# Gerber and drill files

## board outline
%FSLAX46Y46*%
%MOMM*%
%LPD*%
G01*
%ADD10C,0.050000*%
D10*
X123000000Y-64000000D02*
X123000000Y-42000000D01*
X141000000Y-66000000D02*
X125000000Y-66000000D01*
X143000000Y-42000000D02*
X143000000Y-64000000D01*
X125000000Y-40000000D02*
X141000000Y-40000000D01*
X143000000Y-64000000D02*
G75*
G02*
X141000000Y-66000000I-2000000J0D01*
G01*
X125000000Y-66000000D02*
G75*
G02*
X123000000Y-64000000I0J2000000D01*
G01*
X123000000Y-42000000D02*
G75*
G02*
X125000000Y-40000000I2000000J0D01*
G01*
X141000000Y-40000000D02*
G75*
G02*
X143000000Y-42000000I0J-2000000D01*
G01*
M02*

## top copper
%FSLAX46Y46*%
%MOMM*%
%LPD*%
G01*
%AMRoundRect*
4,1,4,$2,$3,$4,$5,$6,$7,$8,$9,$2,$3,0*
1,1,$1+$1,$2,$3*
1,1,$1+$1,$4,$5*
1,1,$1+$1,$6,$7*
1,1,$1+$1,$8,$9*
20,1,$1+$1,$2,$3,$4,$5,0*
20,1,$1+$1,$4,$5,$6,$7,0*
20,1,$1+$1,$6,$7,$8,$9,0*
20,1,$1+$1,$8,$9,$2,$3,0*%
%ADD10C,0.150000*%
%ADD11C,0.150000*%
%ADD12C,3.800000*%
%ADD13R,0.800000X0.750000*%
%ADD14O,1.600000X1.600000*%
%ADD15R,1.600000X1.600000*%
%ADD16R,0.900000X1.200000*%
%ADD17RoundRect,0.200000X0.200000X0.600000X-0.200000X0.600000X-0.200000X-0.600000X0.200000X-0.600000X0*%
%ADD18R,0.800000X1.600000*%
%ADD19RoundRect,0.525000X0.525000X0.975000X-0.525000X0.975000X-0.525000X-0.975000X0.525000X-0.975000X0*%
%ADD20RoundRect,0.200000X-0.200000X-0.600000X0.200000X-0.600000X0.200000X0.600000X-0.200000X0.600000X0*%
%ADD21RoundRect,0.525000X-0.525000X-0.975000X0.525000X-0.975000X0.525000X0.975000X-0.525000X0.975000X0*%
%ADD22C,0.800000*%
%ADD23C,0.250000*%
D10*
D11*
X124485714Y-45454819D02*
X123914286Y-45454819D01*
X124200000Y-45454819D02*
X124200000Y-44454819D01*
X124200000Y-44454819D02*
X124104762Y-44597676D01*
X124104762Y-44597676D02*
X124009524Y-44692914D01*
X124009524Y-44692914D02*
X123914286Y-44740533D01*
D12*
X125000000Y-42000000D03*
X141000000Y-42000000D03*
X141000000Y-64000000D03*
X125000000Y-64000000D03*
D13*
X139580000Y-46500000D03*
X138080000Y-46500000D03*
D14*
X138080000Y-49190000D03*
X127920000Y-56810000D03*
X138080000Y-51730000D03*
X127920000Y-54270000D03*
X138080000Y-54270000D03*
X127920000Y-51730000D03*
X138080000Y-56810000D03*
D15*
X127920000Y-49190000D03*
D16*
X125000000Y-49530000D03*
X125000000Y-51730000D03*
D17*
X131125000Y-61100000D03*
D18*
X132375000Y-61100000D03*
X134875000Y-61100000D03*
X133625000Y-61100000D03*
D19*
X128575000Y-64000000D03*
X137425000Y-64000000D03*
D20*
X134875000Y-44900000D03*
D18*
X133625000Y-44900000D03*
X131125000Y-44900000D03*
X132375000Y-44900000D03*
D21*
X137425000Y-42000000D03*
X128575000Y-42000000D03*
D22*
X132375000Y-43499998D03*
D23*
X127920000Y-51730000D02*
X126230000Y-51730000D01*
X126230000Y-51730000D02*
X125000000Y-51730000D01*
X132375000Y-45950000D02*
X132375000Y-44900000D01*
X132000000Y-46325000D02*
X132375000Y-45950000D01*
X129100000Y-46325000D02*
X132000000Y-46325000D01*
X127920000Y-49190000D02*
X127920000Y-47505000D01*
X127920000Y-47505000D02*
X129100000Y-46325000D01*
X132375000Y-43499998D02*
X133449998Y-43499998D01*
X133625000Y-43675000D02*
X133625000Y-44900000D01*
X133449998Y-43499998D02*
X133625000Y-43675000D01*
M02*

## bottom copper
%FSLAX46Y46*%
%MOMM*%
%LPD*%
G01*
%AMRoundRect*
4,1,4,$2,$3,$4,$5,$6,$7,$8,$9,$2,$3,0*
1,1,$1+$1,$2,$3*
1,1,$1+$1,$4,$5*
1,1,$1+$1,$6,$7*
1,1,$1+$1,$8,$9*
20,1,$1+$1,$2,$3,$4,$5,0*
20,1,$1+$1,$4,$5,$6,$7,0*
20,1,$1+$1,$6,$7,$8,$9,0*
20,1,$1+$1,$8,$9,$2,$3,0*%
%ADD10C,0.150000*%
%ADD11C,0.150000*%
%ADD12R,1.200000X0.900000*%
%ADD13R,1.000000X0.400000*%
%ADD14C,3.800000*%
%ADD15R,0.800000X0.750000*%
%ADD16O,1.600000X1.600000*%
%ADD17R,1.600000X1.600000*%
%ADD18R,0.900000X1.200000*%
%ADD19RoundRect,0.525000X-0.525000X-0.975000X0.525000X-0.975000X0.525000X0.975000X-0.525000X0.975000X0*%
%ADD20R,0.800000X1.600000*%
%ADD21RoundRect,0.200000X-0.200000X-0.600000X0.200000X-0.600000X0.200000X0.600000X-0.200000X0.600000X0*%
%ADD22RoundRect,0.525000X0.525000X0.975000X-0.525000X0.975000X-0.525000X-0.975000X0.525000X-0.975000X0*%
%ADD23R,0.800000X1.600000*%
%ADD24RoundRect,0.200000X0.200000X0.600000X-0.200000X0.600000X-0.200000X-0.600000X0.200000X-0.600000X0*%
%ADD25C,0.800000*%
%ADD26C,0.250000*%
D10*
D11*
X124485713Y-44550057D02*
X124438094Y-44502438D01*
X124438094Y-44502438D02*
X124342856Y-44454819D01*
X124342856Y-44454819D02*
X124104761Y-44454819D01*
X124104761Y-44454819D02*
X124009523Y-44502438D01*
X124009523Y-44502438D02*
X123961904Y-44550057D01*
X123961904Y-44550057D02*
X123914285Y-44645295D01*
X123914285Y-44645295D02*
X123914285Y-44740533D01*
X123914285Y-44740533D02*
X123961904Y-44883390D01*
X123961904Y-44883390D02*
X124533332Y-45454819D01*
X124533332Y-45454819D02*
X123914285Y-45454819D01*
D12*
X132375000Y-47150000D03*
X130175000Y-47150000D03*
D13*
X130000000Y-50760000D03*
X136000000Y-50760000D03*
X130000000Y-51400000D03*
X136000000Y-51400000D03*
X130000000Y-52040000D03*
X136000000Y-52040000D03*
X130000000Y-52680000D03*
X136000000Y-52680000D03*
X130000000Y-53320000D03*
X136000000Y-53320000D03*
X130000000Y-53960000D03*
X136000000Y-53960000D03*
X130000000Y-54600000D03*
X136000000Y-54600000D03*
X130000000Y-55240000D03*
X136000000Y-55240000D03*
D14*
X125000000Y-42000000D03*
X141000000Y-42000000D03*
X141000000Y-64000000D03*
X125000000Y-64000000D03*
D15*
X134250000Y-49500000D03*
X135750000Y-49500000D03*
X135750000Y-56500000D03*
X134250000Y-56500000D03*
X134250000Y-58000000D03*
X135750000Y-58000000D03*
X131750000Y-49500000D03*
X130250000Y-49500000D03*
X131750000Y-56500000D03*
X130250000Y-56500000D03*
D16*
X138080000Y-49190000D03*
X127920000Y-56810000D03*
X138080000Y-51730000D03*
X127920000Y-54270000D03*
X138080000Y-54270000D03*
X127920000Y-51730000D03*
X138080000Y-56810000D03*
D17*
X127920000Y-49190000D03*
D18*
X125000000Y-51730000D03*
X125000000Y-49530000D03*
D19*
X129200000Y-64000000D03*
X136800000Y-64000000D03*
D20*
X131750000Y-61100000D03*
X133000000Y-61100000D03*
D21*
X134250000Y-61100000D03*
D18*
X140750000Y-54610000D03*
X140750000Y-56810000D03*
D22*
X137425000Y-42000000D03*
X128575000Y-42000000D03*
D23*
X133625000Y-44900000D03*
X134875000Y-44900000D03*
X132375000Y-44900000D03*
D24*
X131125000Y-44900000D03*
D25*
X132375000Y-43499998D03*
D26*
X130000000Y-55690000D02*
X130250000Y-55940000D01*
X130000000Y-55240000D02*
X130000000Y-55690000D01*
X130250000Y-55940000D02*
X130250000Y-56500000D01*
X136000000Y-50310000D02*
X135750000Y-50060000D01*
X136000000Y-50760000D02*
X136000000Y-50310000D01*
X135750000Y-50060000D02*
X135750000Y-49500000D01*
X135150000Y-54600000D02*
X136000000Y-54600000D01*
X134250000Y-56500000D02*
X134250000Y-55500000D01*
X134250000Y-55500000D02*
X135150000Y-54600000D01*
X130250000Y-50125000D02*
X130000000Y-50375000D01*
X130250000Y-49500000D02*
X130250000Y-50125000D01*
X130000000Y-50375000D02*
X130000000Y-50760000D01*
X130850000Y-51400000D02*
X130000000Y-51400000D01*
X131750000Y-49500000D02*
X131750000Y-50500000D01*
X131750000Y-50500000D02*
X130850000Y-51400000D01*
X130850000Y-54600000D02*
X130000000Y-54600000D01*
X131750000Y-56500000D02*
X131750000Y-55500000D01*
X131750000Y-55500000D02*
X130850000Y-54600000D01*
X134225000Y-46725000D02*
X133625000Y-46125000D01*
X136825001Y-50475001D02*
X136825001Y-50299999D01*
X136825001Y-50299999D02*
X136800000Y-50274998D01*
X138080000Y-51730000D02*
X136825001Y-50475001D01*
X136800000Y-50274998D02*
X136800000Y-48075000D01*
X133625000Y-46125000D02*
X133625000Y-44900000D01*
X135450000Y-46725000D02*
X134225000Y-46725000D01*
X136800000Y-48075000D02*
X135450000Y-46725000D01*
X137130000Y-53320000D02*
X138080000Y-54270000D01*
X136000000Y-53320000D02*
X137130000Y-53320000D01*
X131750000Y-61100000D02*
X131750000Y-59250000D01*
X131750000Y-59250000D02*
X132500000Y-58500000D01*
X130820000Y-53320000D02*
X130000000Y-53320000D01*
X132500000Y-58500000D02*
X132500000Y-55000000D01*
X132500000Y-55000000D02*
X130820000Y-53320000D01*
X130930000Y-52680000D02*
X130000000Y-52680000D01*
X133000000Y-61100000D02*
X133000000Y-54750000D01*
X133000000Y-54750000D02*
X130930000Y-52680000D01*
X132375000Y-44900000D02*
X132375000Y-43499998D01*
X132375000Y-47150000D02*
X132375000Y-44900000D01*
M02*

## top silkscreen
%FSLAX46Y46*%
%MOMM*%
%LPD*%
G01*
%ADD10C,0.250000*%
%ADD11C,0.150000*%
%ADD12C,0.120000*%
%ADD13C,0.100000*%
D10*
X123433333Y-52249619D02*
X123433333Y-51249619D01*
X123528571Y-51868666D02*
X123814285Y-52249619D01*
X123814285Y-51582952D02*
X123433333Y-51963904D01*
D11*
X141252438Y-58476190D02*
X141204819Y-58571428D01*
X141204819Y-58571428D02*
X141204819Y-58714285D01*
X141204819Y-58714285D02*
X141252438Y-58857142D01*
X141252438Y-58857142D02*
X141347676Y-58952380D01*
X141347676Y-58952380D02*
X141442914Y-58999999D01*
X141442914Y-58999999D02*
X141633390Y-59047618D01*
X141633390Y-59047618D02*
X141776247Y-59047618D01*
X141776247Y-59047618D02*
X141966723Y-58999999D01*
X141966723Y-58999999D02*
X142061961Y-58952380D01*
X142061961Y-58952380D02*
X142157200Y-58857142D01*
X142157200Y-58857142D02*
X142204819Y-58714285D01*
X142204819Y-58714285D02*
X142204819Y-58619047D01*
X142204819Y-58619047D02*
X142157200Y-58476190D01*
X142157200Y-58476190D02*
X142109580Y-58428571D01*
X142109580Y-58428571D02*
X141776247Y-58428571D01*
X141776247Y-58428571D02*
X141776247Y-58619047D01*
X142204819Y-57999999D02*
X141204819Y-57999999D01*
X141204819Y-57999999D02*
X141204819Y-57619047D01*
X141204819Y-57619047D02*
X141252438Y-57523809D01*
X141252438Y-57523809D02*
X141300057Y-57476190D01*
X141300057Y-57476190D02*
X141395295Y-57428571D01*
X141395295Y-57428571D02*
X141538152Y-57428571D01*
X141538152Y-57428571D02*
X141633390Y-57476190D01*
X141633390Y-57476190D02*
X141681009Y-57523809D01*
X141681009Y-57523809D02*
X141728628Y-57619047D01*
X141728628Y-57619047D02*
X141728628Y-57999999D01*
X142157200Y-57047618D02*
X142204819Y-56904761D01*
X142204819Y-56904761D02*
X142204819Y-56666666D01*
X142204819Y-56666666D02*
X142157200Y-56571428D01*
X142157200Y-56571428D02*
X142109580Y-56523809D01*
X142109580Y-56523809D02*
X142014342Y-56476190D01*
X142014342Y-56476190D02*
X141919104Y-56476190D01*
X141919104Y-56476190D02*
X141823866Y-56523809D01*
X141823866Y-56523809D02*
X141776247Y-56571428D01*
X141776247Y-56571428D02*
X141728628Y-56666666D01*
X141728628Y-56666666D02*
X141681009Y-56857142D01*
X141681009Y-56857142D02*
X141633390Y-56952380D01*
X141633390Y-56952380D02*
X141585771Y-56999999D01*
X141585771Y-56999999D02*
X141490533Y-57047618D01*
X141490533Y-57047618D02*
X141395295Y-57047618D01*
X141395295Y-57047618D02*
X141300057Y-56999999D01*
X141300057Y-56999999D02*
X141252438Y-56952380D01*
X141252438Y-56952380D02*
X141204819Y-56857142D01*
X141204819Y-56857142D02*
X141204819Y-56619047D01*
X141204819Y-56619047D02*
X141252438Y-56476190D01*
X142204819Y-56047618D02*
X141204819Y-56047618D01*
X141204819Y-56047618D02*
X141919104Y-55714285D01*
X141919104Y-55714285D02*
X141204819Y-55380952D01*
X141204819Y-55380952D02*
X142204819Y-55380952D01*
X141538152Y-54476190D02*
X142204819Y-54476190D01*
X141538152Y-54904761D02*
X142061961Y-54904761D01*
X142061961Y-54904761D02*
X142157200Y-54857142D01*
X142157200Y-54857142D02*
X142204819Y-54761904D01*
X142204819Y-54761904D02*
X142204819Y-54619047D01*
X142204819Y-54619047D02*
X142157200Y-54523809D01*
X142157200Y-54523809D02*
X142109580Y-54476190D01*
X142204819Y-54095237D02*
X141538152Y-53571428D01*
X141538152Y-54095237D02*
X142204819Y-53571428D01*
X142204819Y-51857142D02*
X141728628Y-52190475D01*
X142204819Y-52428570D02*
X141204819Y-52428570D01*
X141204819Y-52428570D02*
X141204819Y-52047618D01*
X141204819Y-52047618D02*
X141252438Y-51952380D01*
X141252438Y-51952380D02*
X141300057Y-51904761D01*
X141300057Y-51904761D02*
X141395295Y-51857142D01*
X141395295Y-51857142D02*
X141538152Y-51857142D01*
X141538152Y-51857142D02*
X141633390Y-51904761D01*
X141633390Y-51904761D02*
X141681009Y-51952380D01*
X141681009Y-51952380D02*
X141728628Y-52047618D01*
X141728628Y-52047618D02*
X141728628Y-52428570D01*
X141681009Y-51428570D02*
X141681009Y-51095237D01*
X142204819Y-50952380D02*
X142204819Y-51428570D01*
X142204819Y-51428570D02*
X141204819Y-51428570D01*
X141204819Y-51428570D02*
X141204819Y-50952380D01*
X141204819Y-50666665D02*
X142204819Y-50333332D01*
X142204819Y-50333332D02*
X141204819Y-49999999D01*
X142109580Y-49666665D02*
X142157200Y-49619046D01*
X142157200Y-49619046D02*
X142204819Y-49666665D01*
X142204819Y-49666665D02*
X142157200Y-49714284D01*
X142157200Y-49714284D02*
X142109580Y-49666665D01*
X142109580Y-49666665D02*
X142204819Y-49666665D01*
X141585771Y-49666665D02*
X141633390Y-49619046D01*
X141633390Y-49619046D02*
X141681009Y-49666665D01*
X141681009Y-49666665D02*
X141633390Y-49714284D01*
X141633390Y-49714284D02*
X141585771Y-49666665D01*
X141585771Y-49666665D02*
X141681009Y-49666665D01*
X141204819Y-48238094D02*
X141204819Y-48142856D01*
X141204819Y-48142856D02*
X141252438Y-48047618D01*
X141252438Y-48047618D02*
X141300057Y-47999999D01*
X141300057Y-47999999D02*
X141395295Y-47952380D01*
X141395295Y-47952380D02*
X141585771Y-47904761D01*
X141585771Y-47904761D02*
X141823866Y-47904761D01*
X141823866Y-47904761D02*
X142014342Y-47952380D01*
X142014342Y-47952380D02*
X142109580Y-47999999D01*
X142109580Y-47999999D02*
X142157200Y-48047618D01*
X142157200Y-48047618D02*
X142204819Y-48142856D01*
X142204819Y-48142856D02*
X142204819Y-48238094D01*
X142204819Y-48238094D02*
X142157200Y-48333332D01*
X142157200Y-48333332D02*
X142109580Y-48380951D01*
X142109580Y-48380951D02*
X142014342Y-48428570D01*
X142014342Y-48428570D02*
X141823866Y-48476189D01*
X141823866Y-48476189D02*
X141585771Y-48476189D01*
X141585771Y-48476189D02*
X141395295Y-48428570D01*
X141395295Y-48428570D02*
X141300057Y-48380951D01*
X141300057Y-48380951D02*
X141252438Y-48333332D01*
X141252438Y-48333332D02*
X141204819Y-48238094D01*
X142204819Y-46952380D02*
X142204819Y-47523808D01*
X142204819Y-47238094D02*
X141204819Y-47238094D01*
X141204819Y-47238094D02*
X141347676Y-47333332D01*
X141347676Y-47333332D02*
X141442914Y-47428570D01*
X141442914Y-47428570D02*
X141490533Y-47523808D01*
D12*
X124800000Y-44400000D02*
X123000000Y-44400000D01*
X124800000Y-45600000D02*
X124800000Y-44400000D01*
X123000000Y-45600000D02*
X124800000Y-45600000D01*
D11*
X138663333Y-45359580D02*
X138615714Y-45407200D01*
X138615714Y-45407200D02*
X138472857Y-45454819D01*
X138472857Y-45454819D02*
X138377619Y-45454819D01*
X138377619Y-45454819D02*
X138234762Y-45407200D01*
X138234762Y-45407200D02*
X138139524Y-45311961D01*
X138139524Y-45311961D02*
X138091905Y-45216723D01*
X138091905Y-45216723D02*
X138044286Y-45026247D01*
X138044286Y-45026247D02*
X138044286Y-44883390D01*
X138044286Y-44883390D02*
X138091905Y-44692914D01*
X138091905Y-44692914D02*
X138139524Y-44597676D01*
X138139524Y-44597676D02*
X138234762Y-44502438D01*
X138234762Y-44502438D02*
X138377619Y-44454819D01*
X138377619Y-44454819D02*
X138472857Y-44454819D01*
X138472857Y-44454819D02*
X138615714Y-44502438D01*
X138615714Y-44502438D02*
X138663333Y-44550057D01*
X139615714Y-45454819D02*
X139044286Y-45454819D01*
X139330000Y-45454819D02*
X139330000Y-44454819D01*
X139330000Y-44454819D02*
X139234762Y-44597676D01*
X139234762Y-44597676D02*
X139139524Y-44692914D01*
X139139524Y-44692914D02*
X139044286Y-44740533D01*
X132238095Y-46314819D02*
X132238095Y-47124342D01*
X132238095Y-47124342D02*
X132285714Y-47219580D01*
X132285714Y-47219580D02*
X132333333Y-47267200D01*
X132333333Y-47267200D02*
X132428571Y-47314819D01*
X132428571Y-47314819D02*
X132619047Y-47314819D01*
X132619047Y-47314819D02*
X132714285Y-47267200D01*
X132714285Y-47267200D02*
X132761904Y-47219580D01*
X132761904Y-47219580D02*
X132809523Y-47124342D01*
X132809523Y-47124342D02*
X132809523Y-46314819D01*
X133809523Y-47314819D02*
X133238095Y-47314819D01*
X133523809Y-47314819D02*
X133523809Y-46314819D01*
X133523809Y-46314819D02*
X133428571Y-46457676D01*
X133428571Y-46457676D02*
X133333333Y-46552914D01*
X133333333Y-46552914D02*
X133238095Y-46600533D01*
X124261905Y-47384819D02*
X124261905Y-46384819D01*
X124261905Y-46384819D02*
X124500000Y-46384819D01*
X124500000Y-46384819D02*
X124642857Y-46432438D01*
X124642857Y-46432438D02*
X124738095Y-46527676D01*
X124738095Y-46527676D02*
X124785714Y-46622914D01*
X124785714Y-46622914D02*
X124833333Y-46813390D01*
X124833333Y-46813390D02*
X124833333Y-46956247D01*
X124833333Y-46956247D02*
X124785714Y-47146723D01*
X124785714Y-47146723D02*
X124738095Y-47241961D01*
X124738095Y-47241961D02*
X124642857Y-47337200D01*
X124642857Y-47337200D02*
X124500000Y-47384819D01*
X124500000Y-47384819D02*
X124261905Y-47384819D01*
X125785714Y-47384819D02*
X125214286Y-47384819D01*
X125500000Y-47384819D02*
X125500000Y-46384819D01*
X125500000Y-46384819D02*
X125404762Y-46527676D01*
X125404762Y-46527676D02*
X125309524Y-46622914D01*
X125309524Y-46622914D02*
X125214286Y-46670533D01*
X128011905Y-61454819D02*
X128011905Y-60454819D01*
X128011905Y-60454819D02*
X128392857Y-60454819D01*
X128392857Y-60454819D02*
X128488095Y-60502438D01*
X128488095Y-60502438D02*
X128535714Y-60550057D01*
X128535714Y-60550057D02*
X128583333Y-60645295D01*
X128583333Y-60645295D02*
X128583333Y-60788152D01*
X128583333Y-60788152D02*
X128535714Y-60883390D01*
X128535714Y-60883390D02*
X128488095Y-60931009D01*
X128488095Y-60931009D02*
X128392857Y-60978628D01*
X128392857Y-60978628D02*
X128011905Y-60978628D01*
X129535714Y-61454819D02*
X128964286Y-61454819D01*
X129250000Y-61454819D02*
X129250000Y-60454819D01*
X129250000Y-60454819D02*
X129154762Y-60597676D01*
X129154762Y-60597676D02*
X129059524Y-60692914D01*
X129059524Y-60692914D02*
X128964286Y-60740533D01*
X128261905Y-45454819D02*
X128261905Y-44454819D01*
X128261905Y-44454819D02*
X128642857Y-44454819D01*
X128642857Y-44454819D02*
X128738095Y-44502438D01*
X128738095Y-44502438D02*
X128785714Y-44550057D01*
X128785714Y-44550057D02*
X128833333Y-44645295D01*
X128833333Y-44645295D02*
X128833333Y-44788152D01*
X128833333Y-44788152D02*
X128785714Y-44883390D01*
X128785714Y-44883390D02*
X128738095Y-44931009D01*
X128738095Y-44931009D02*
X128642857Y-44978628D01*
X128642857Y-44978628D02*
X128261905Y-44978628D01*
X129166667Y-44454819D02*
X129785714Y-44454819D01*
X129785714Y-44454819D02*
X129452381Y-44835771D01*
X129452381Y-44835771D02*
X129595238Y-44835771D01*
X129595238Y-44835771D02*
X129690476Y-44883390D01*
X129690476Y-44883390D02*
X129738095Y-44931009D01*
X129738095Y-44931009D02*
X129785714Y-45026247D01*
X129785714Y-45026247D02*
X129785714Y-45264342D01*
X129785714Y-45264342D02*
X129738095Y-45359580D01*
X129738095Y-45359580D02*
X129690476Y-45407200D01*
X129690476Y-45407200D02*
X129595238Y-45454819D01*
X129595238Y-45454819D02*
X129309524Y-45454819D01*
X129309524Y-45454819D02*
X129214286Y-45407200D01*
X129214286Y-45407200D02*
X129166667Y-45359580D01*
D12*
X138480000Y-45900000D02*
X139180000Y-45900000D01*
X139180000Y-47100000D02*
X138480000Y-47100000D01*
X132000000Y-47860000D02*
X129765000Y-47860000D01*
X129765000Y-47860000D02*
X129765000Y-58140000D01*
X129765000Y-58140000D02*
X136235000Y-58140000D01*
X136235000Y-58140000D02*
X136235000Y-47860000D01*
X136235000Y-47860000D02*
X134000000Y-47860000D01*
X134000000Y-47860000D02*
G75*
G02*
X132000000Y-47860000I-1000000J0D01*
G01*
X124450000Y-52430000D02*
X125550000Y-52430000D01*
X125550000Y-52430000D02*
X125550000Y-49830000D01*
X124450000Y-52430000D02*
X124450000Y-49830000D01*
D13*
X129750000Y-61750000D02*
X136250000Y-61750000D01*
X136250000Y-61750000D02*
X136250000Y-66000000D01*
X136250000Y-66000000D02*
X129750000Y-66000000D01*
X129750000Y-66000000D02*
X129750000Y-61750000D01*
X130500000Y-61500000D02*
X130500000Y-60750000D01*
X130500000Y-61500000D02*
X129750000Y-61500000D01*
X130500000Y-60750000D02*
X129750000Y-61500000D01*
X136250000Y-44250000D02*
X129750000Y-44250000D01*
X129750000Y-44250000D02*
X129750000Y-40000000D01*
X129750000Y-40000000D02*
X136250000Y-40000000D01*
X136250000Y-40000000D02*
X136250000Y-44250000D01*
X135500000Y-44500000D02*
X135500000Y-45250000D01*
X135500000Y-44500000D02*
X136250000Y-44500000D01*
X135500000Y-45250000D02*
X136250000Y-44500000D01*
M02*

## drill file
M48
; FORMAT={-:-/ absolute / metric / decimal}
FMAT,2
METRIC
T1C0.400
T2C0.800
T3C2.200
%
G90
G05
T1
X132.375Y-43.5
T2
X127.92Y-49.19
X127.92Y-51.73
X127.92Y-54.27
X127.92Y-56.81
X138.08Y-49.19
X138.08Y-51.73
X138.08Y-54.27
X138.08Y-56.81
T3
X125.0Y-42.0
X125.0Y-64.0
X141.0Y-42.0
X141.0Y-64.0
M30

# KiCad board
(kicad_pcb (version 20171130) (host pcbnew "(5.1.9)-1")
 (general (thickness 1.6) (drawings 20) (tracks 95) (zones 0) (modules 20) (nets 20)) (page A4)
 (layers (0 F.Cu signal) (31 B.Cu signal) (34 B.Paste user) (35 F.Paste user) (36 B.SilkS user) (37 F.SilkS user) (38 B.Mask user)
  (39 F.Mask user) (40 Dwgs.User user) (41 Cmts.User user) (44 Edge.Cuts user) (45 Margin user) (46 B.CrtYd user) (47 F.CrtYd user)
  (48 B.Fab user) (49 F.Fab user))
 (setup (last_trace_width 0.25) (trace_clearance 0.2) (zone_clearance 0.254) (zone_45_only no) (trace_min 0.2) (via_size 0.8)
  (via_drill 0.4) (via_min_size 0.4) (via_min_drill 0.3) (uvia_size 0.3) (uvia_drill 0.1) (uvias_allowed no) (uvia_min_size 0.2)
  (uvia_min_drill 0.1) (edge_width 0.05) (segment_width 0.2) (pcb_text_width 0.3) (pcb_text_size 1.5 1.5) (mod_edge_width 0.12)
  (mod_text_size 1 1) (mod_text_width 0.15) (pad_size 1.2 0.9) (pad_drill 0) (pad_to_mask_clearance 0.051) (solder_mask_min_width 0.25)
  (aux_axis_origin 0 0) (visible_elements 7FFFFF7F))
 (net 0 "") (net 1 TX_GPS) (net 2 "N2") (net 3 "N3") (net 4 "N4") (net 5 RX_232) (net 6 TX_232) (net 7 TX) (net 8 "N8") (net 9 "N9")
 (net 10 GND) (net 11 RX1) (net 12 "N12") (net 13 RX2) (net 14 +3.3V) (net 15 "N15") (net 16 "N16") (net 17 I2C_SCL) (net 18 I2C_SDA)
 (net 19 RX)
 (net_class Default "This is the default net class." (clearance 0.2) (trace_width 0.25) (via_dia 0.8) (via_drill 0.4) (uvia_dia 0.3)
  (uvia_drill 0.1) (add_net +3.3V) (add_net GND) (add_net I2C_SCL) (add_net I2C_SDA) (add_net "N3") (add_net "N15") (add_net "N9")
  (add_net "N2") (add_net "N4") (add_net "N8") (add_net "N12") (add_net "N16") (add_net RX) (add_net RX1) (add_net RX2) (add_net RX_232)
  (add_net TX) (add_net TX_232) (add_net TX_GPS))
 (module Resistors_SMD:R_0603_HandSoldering (layer B.Cu) (at 131.275 47.15 180)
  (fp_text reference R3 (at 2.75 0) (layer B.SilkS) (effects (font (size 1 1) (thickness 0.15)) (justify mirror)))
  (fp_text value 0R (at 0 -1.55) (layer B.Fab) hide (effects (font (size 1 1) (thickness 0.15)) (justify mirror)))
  (pad 1 smd rect (at -1.1 0 180) (size 1.2 0.9) (layers B.Cu B.Paste B.Mask) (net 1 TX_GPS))
  (pad 2 smd rect (at 1.1 0 180) (size 1.2 0.9) (layers B.Cu B.Paste B.Mask)))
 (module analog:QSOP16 (layer B.Cu) (at 133 53 270) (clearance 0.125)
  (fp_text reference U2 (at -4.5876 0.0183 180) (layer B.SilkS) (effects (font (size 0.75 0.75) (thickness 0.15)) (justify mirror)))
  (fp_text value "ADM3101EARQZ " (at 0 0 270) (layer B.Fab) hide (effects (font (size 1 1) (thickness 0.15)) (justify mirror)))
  (pad 16 smd rect (at -2.24 3 270) (size 0.4 1) (layers B.Cu B.Paste B.Mask) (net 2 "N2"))
  (pad 1 smd rect (at -2.24 -3 270) (size 0.4 1) (layers B.Cu B.Paste B.Mask) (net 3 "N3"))
  (pad 15 smd rect (at -1.6 3 270) (size 0.4 1) (layers B.Cu B.Paste B.Mask) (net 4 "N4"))
  (pad 2 smd rect (at -1.6 -3 270) (size 0.4 1) (layers B.Cu B.Paste B.Mask))
  (pad 14 smd rect (at -0.96 3 270) (size 0.4 1) (layers B.Cu B.Paste B.Mask))
  (pad 3 smd rect (at -0.96 -3 270) (size 0.4 1) (layers B.Cu B.Paste B.Mask))
  (pad 13 smd rect (at -0.32 3 270) (size 0.4 1) (layers B.Cu B.Paste B.Mask) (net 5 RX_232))
  (pad 4 smd rect (at -0.32 -3 270) (size 0.4 1) (layers B.Cu B.Paste B.Mask))
  (pad 12 smd rect (at 0.32 3 270) (size 0.4 1) (layers B.Cu B.Paste B.Mask) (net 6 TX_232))
  (pad 5 smd rect (at 0.32 -3 270) (size 0.4 1) (layers B.Cu B.Paste B.Mask) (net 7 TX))
  (pad 11 smd rect (at 0.96 3 270) (size 0.4 1) (layers B.Cu B.Paste B.Mask))
  (pad 6 smd rect (at 0.96 -3 270) (size 0.4 1) (layers B.Cu B.Paste B.Mask))
  (pad 10 smd rect (at 1.6 3 270) (size 0.4 1) (layers B.Cu B.Paste B.Mask) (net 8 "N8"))
  (pad 7 smd rect (at 1.6 -3 270) (size 0.4 1) (layers B.Cu B.Paste B.Mask) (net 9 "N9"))
  (pad 9 smd rect (at 2.24 3 270) (size 0.4 1) (layers B.Cu B.Paste B.Mask) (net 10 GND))
  (pad 8 smd rect (at 2.24 -3 270) (size 0.4 1) (layers B.Cu B.Paste B.Mask)))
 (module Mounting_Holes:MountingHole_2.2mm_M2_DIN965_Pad (layer F.Cu) (at 125 42)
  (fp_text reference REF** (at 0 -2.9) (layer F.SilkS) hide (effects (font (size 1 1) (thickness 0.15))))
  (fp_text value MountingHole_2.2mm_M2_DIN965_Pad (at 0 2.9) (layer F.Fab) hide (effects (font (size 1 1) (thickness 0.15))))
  (pad 1 thru_hole circle (at 0 0) (size 3.8 3.8) (drill 2.2) (layers *.Cu *.Mask)))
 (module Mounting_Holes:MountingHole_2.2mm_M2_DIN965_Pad (layer F.Cu) (at 141 42)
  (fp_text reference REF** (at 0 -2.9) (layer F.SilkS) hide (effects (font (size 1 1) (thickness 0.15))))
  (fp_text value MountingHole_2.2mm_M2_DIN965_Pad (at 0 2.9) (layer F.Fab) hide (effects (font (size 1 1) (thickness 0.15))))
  (pad 1 thru_hole circle (at 0 0) (size 3.8 3.8) (drill 2.2) (layers *.Cu *.Mask)))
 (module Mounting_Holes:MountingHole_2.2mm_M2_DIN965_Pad (layer F.Cu) (at 141 64)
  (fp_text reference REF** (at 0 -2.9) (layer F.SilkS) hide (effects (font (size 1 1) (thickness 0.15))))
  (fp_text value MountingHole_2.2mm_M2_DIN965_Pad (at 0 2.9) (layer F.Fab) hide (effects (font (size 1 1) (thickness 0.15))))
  (pad 1 thru_hole circle (at 0 0) (size 3.8 3.8) (drill 2.2) (layers *.Cu *.Mask)))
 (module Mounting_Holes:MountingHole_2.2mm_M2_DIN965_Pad (layer F.Cu) (at 125 64)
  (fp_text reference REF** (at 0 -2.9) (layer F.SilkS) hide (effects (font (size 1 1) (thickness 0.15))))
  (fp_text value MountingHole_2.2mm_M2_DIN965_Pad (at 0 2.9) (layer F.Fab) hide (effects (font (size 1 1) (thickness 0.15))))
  (pad 1 thru_hole circle (at 0 0) (size 3.8 3.8) (drill 2.2) (layers *.Cu *.Mask)))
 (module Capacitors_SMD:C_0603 (layer F.Cu) (at 138.83 46.5)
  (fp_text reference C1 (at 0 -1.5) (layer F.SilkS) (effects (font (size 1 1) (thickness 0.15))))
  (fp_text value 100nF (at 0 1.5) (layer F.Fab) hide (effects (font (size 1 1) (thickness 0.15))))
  (fp_line (start -0.35 -0.6) (end 0.35 -0.6) (layer F.SilkS) (width 0.12))
  (fp_line (start 0.35 0.6) (end -0.35 0.6) (layer F.SilkS) (width 0.12))
  (pad 2 smd rect (at 0.75 0) (size 0.8 0.75) (layers F.Cu F.Paste F.Mask))
  (pad 1 smd rect (at -0.75 0) (size 0.8 0.75) (layers F.Cu F.Paste F.Mask)))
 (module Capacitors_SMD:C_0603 (layer B.Cu) (at 135 49.5 180)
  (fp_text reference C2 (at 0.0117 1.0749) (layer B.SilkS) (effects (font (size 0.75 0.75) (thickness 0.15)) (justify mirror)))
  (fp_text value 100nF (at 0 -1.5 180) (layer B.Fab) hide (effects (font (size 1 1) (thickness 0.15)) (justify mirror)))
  (pad 2 smd rect (at 0.75 0 180) (size 0.8 0.75) (layers B.Cu B.Paste B.Mask))
  (pad 1 smd rect (at -0.75 0 180) (size 0.8 0.75) (layers B.Cu B.Paste B.Mask) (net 3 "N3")))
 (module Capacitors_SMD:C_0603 (layer B.Cu) (at 135 56.5)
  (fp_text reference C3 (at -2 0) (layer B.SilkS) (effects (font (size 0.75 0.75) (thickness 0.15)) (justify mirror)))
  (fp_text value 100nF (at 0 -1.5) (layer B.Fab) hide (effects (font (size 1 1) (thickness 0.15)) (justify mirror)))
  (pad 2 smd rect (at 0.75 0) (size 0.8 0.75) (layers B.Cu B.Paste B.Mask))
  (pad 1 smd rect (at -0.75 0) (size 0.8 0.75) (layers B.Cu B.Paste B.Mask) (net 9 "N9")))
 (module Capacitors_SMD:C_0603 (layer B.Cu) (at 135 58 180)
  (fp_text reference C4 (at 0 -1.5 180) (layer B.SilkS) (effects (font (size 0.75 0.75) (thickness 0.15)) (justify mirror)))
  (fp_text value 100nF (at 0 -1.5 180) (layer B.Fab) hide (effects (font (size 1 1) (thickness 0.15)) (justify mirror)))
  (pad 2 smd rect (at 0.75 0 180) (size 0.8 0.75) (layers B.Cu B.Paste B.Mask))
  (pad 1 smd rect (at -0.75 0 180) (size 0.8 0.75) (layers B.Cu B.Paste B.Mask)))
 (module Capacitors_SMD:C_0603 (layer B.Cu) (at 131 49.5)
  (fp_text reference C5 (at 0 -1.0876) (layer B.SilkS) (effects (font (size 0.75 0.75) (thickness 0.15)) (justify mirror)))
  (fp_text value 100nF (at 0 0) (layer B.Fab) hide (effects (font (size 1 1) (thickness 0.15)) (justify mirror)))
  (pad 2 smd rect (at 0.75 0) (size 0.8 0.75) (layers B.Cu B.Paste B.Mask) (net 4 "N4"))
  (pad 1 smd rect (at -0.75 0) (size 0.8 0.75) (layers B.Cu B.Paste B.Mask) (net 2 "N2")))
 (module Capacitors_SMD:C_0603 (layer B.Cu) (at 131 56.5)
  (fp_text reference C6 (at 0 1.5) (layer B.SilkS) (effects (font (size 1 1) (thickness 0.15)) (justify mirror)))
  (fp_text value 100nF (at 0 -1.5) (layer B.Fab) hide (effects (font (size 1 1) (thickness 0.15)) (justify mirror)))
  (pad 2 smd rect (at 0.75 0) (size 0.8 0.75) (layers B.Cu B.Paste B.Mask) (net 8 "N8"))
  (pad 1 smd rect (at -0.75 0) (size 0.8 0.75) (layers B.Cu B.Paste B.Mask) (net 10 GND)))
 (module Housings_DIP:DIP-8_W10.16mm (layer F.Cu) (at 133 53)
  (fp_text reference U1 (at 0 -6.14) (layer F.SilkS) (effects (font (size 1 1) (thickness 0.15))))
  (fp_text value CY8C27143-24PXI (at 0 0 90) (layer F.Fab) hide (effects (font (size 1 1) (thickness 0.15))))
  (fp_line (start -1 -5.14) (end -3.235 -5.14) (layer F.SilkS) (width 0.12))
  (fp_line (start -3.235 -5.14) (end -3.235 5.14) (layer F.SilkS) (width 0.12))
  (fp_line (start -3.235 5.14) (end 3.235 5.14) (layer F.SilkS) (width 0.12))
  (fp_line (start 3.235 5.14) (end 3.235 -5.14) (layer F.SilkS) (width 0.12))
  (fp_line (start 3.235 -5.14) (end 1 -5.14) (layer F.SilkS) (width 0.12))
  (fp_arc (start 0 -5.14) (end -1 -5.14) (angle -180) (layer F.SilkS) (width 0.12))
  (pad 8 thru_hole oval (at 5.08 -3.81) (size 1.6 1.6) (drill 0.8) (layers *.Cu *.Mask))
  (pad 4 thru_hole oval (at -5.08 3.81) (size 1.6 1.6) (drill 0.8) (layers *.Cu *.Mask))
  (pad 7 thru_hole oval (at 5.08 -1.27) (size 1.6 1.6) (drill 0.8) (layers *.Cu *.Mask) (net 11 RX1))
  (pad 3 thru_hole oval (at -5.08 1.27) (size 1.6 1.6) (drill 0.8) (layers *.Cu *.Mask))
  (pad 6 thru_hole oval (at 5.08 1.27) (size 1.6 1.6) (drill 0.8) (layers *.Cu *.Mask) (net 7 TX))
  (pad 2 thru_hole oval (at -5.08 -1.27) (size 1.6 1.6) (drill 0.8) (layers *.Cu *.Mask) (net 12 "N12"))
  (pad 5 thru_hole oval (at 5.08 3.81) (size 1.6 1.6) (drill 0.8) (layers *.Cu *.Mask))
  (pad 1 thru_hole rect (at -5.08 -3.81) (size 1.6 1.6) (drill 0.8) (layers *.Cu *.Mask) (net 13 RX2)))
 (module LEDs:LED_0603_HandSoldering (layer F.Cu) (at 125 50.63 90)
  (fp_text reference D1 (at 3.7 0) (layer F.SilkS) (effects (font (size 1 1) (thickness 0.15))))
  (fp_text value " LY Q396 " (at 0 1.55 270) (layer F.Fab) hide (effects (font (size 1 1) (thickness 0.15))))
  (fp_line (start -1.8 -0.55) (end -1.8 0.55) (layer F.SilkS) (width 0.12))
  (fp_line (start -1.8 0.55) (end 0.8 0.55) (layer F.SilkS) (width 0.12))
  (fp_line (start -1.8 -0.55) (end 0.8 -0.55) (layer F.SilkS) (width 0.12))
  (pad 2 smd rect (at 1.1 0 90) (size 1.2 0.9) (layers F.Cu F.Paste F.Mask))
  (pad 1 smd rect (at -1.1 0 90) (size 1.2 0.9) (layers F.Cu F.Paste F.Mask) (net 12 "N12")))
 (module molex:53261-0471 (layer F.Cu) (at 133 64 180) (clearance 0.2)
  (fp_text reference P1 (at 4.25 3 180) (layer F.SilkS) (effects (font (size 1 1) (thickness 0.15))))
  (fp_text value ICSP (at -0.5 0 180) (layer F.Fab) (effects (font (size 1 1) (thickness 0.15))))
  (fp_line (start 3.25 2.25) (end -3.25 2.25) (layer F.SilkS) (width 0.1))
  (fp_line (start -3.25 2.25) (end -3.25 -2) (layer F.SilkS) (width 0.1))
  (fp_line (start -3.25 -2) (end 3.25 -2) (layer F.SilkS) (width 0.1))
  (fp_line (start 3.25 -2) (end 3.25 2.25) (layer F.SilkS) (width 0.1))
  (fp_line (start 2.5 2.5) (end 2.5 3.25) (layer F.SilkS) (width 0.1))
  (fp_line (start 2.5 2.5) (end 3.25 2.5) (layer F.SilkS) (width 0.1))
  (fp_line (start 2.5 3.25) (end 3.25 2.5) (layer F.SilkS) (width 0.1))
  (pad 1 connect roundrect (at 1.875 2.9 180) (size 0.8 1.6) (layers F.Cu F.Mask) (roundrect_rratio 0.25))
  (pad 2 connect rect (at 0.625 2.9 180) (size 0.8 1.6) (layers F.Cu F.Mask))
  (pad 4 connect rect (at -1.875 2.9 180) (size 0.8 1.6) (layers F.Cu F.Mask))
  (pad 3 connect rect (at -0.625 2.9 180) (size 0.8 1.6) (layers F.Cu F.Mask))
  (pad "" connect roundrect (at 4.425 0 180) (size 2.1 3) (layers F.Cu F.Mask) (roundrect_rratio 0.25))
  (pad "" connect roundrect (at -4.425 0 180) (size 2.1 3) (layers F.Cu F.Mask) (roundrect_rratio 0.25)))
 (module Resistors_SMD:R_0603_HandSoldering (layer B.Cu) (at 125 50.63 270)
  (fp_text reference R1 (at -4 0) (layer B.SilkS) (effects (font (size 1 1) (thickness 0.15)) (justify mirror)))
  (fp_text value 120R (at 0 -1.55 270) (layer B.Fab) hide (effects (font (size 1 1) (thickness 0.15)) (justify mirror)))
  (pad 2 smd rect (at 1.1 0 270) (size 1.2 0.9) (layers B.Cu B.Paste B.Mask))
  (pad 1 smd rect (at -1.1 0 270) (size 1.2 0.9) (layers B.Cu B.Paste B.Mask)))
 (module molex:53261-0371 (layer B.Cu) (at 133 64) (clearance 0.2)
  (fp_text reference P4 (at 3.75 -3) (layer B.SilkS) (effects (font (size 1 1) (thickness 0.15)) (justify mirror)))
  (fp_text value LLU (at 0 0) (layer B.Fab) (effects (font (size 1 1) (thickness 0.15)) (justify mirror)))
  (pad "" connect roundrect (at -3.8 0) (size 2.1 3) (layers B.Cu B.Mask) (roundrect_rratio 0.25))
  (pad "" connect roundrect (at 3.8 0) (size 2.1 3) (layers B.Cu B.Mask) (roundrect_rratio 0.25))
  (pad 3 smd rect (at -1.25 -2.9) (size 0.8 1.6) (layers B.Cu B.Paste B.Mask) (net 6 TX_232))
  (pad 2 smd rect (at 0 -2.9) (size 0.8 1.6) (layers B.Cu B.Paste B.Mask) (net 5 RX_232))
  (pad 1 smd roundrect (at 1.25 -2.9) (size 0.8 1.6) (layers B.Cu B.Paste B.Mask) (roundrect_rratio 0.25)))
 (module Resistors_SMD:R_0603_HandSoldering (layer B.Cu) (at 140.75 55.71 90)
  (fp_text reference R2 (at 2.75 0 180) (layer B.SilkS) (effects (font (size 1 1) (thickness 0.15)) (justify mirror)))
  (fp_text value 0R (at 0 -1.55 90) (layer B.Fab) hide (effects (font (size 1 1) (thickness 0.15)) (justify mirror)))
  (pad 2 smd rect (at 1.1 0 90) (size 1.2 0.9) (layers B.Cu B.Paste B.Mask))
  (pad 1 smd rect (at -1.1 0 90) (size 1.2 0.9) (layers B.Cu B.Paste B.Mask)))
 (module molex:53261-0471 (layer B.Cu) (at 133 42 180) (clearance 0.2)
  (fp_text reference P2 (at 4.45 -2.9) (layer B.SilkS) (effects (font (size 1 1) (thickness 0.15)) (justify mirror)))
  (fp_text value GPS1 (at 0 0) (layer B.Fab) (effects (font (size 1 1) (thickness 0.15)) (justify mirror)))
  (pad "" connect roundrect (at -4.425 0 180) (size 2.1 3) (layers B.Cu B.Mask) (roundrect_rratio 0.25))
  (pad "" connect roundrect (at 4.425 0 180) (size 2.1 3) (layers B.Cu B.Mask) (roundrect_rratio 0.25))
  (pad 3 connect rect (at -0.625 -2.9 180) (size 0.8 1.6) (layers B.Cu B.Mask) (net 11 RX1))
  (pad 4 connect rect (at -1.875 -2.9 180) (size 0.8 1.6) (layers B.Cu B.Mask))
  (pad 2 connect rect (at 0.625 -2.9 180) (size 0.8 1.6) (layers B.Cu B.Mask) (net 1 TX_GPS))
  (pad 1 connect roundrect (at 1.875 -2.9 180) (size 0.8 1.6) (layers B.Cu B.Mask) (roundrect_rratio 0.25)))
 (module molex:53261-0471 (layer F.Cu) (at 133 42) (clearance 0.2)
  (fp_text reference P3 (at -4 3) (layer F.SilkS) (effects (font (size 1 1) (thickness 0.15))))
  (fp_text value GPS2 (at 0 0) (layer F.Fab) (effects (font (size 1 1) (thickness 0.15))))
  (fp_line (start 3.25 2.25) (end -3.25 2.25) (layer F.SilkS) (width 0.1))
  (fp_line (start -3.25 2.25) (end -3.25 -2) (layer F.SilkS) (width 0.1))
  (fp_line (start -3.25 -2) (end 3.25 -2) (layer F.SilkS) (width 0.1))
  (fp_line (start 3.25 -2) (end 3.25 2.25) (layer F.SilkS) (width 0.1))
  (fp_line (start 2.5 2.5) (end 2.5 3.25) (layer F.SilkS) (width 0.1))
  (fp_line (start 2.5 2.5) (end 3.25 2.5) (layer F.SilkS) (width 0.1))
  (fp_line (start 2.5 3.25) (end 3.25 2.5) (layer F.SilkS) (width 0.1))
  (pad 1 connect roundrect (at 1.875 2.9) (size 0.8 1.6) (layers F.Cu F.Mask) (roundrect_rratio 0.25))
  (pad 2 connect rect (at 0.625 2.9) (size 0.8 1.6) (layers F.Cu F.Mask) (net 1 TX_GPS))
  (pad 4 connect rect (at -1.875 2.9) (size 0.8 1.6) (layers F.Cu F.Mask))
  (pad 3 connect rect (at -0.625 2.9) (size 0.8 1.6) (layers F.Cu F.Mask) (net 13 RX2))
  (pad "" connect roundrect (at 4.425 0) (size 2.1 3) (layers F.Cu F.Mask) (roundrect_rratio 0.25))
  (pad "" connect roundrect (at -4.425 0) (size 2.1 3) (layers F.Cu F.Mask) (roundrect_rratio 0.25)))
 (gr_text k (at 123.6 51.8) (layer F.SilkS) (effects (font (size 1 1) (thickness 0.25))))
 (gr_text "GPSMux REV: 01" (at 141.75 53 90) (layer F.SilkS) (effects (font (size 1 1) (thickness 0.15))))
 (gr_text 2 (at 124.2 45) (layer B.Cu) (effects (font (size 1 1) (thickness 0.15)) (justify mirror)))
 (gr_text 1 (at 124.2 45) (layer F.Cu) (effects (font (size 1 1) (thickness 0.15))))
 (gr_line (start 124.8 44.4) (end 123 44.4) (layer F.SilkS) (width 0.12))
 (gr_line (start 124.8 45.6) (end 124.8 44.4) (layer F.SilkS) (width 0.12))
 (gr_line (start 123 45.6) (end 124.8 45.6) (layer F.SilkS) (width 0.12))
 (gr_line (start 123 64) (end 123 42) (layer Edge.Cuts) (width 0.05))
 (gr_line (start 141 66) (end 125 66) (layer Edge.Cuts) (width 0.05))
 (gr_line (start 143 42) (end 143 64) (layer Edge.Cuts) (width 0.05))
 (gr_line (start 125 40) (end 141 40) (layer Edge.Cuts) (width 0.05))
 (gr_arc (start 141 64) (end 141 66) (angle -90) (layer Edge.Cuts) (width 0.05))
 (gr_arc (start 125 64) (end 123 64) (angle -90) (layer Edge.Cuts) (width 0.05))
 (gr_arc (start 125 42) (end 125 40) (angle -90) (layer Edge.Cuts) (width 0.05))
 (gr_arc (start 141 42) (end 143 42) (angle -90) (layer Edge.Cuts) (width 0.05))
 (via (at 132.375 43.499998) (size 0.8) (layers F.Cu B.Cu) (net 1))
 (segment (start 130 55.69) (end 130.25 55.94) (width 0.25) (layer B.Cu) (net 10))
 (segment (start 130 55.24) (end 130 55.69) (width 0.25) (layer B.Cu) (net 10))
 (segment (start 130.25 55.94) (end 130.25 56.5) (width 0.25) (layer B.Cu) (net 10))
 (segment (start 136 50.31) (end 135.75 50.06) (width 0.25) (layer B.Cu) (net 3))
 (segment (start 136 50.76) (end 136 50.31) (width 0.25) (layer B.Cu) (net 3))
 (segment (start 135.75 50.06) (end 135.75 49.5) (width 0.25) (layer B.Cu) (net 3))
 (segment (start 135.15 54.6) (end 136 54.6) (width 0.25) (layer B.Cu) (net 9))
 (segment (start 134.25 56.5) (end 134.25 55.5) (width 0.25) (layer B.Cu) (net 9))
 (segment (start 134.25 55.5) (end 135.15 54.6) (width 0.25) (layer B.Cu) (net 9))
 (segment (start 130.25 50.125) (end 130 50.375) (width 0.25) (layer B.Cu) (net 2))
 (segment (start 130.25 49.5) (end 130.25 50.125) (width 0.25) (layer B.Cu) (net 2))
 (segment (start 130 50.375) (end 130 50.76) (width 0.25) (layer B.Cu) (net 2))
 (segment (start 130.85 51.4) (end 130 51.4) (width 0.25) (layer B.Cu) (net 4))
 (segment (start 131.75 49.5) (end 131.75 50.5) (width 0.25) (layer B.Cu) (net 4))
 (segment (start 131.75 50.5) (end 130.85 51.4) (width 0.25) (layer B.Cu) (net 4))
 (segment (start 130.85 54.6) (end 130 54.6) (width 0.25) (layer B.Cu) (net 8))
 (segment (start 131.75 56.5) (end 131.75 55.5) (width 0.25) (layer B.Cu) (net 8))
 (segment (start 131.75 55.5) (end 130.85 54.6) (width 0.25) (layer B.Cu) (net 8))
 (segment (start 127.92 51.73) (end 126.23 51.73) (width 0.25) (layer F.Cu) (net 12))
 (segment (start 126.23 51.73) (end 125 51.73) (width 0.25) (layer F.Cu) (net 12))
 (segment (start 134.225 46.725) (end 133.625 46.125) (width 0.25) (layer B.Cu) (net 11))
 (segment (start 136.825001 50.475001) (end 136.825001 50.299999) (width 0.25) (layer B.Cu) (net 11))
 (segment (start 136.825001 50.299999) (end 136.8 50.274998) (width 0.25) (layer B.Cu) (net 11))
 (segment (start 138.08 51.73) (end 136.825001 50.475001) (width 0.25) (layer B.Cu) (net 11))
 (segment (start 136.8 50.274998) (end 136.8 48.075) (width 0.25) (layer B.Cu) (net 11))
 (segment (start 133.625 46.125) (end 133.625 44.9) (width 0.25) (layer B.Cu) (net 11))
 (segment (start 135.45 46.725) (end 134.225 46.725) (width 0.25) (layer B.Cu) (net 11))
 (segment (start 136.8 48.075) (end 135.45 46.725) (width 0.25) (layer B.Cu) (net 11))
 (segment (start 132.375 45.95) (end 132.375 44.9) (width 0.25) (layer F.Cu) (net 13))
 (segment (start 132 46.325) (end 132.375 45.95) (width 0.25) (layer F.Cu) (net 13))
 (segment (start 129.1 46.325) (end 132 46.325) (width 0.25) (layer F.Cu) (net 13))
 (segment (start 127.92 49.19) (end 127.92 47.505) (width 0.25) (layer F.Cu) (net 13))
 (segment (start 127.92 47.505) (end 129.1 46.325) (width 0.25) (layer F.Cu) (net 13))
 (segment (start 137.13 53.32) (end 138.08 54.27) (width 0.25) (layer B.Cu) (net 7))
 (segment (start 136 53.32) (end 137.13 53.32) (width 0.25) (layer B.Cu) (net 7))
 (segment (start 131.75 61.1) (end 131.75 59.25) (width 0.25) (layer B.Cu) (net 6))
 (segment (start 131.75 59.25) (end 132.5 58.5) (width 0.25) (layer B.Cu) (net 6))
 (segment (start 130.82 53.32) (end 130 53.32) (width 0.25) (layer B.Cu) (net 6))
 (segment (start 132.5 58.5) (end 132.5 55) (width 0.25) (layer B.Cu) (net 6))
 (segment (start 132.5 55) (end 130.82 53.32) (width 0.25) (layer B.Cu) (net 6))
 (segment (start 130.93 52.68) (end 130 52.68) (width 0.25) (layer B.Cu) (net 5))
 (segment (start 133 61.1) (end 133 54.75) (width 0.25) (layer B.Cu) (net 5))
 (segment (start 133 54.75) (end 130.93 52.68) (width 0.25) (layer B.Cu) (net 5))
 (segment (start 132.375 44.9) (end 132.375 43.499998) (width 0.25) (layer B.Cu) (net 1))
 (segment (start 132.375 43.499998) (end 133.449998 43.499998) (width 0.25) (layer F.Cu) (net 1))
 (segment (start 133.625 43.675) (end 133.625 44.9) (width 0.25) (layer F.Cu) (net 1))
 (segment (start 133.449998 43.499998) (end 133.625 43.675) (width 0.25) (layer F.Cu) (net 1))
 (segment (start 132.375 47.15) (end 132.375 44.9) (width 0.25) (layer B.Cu) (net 1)))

